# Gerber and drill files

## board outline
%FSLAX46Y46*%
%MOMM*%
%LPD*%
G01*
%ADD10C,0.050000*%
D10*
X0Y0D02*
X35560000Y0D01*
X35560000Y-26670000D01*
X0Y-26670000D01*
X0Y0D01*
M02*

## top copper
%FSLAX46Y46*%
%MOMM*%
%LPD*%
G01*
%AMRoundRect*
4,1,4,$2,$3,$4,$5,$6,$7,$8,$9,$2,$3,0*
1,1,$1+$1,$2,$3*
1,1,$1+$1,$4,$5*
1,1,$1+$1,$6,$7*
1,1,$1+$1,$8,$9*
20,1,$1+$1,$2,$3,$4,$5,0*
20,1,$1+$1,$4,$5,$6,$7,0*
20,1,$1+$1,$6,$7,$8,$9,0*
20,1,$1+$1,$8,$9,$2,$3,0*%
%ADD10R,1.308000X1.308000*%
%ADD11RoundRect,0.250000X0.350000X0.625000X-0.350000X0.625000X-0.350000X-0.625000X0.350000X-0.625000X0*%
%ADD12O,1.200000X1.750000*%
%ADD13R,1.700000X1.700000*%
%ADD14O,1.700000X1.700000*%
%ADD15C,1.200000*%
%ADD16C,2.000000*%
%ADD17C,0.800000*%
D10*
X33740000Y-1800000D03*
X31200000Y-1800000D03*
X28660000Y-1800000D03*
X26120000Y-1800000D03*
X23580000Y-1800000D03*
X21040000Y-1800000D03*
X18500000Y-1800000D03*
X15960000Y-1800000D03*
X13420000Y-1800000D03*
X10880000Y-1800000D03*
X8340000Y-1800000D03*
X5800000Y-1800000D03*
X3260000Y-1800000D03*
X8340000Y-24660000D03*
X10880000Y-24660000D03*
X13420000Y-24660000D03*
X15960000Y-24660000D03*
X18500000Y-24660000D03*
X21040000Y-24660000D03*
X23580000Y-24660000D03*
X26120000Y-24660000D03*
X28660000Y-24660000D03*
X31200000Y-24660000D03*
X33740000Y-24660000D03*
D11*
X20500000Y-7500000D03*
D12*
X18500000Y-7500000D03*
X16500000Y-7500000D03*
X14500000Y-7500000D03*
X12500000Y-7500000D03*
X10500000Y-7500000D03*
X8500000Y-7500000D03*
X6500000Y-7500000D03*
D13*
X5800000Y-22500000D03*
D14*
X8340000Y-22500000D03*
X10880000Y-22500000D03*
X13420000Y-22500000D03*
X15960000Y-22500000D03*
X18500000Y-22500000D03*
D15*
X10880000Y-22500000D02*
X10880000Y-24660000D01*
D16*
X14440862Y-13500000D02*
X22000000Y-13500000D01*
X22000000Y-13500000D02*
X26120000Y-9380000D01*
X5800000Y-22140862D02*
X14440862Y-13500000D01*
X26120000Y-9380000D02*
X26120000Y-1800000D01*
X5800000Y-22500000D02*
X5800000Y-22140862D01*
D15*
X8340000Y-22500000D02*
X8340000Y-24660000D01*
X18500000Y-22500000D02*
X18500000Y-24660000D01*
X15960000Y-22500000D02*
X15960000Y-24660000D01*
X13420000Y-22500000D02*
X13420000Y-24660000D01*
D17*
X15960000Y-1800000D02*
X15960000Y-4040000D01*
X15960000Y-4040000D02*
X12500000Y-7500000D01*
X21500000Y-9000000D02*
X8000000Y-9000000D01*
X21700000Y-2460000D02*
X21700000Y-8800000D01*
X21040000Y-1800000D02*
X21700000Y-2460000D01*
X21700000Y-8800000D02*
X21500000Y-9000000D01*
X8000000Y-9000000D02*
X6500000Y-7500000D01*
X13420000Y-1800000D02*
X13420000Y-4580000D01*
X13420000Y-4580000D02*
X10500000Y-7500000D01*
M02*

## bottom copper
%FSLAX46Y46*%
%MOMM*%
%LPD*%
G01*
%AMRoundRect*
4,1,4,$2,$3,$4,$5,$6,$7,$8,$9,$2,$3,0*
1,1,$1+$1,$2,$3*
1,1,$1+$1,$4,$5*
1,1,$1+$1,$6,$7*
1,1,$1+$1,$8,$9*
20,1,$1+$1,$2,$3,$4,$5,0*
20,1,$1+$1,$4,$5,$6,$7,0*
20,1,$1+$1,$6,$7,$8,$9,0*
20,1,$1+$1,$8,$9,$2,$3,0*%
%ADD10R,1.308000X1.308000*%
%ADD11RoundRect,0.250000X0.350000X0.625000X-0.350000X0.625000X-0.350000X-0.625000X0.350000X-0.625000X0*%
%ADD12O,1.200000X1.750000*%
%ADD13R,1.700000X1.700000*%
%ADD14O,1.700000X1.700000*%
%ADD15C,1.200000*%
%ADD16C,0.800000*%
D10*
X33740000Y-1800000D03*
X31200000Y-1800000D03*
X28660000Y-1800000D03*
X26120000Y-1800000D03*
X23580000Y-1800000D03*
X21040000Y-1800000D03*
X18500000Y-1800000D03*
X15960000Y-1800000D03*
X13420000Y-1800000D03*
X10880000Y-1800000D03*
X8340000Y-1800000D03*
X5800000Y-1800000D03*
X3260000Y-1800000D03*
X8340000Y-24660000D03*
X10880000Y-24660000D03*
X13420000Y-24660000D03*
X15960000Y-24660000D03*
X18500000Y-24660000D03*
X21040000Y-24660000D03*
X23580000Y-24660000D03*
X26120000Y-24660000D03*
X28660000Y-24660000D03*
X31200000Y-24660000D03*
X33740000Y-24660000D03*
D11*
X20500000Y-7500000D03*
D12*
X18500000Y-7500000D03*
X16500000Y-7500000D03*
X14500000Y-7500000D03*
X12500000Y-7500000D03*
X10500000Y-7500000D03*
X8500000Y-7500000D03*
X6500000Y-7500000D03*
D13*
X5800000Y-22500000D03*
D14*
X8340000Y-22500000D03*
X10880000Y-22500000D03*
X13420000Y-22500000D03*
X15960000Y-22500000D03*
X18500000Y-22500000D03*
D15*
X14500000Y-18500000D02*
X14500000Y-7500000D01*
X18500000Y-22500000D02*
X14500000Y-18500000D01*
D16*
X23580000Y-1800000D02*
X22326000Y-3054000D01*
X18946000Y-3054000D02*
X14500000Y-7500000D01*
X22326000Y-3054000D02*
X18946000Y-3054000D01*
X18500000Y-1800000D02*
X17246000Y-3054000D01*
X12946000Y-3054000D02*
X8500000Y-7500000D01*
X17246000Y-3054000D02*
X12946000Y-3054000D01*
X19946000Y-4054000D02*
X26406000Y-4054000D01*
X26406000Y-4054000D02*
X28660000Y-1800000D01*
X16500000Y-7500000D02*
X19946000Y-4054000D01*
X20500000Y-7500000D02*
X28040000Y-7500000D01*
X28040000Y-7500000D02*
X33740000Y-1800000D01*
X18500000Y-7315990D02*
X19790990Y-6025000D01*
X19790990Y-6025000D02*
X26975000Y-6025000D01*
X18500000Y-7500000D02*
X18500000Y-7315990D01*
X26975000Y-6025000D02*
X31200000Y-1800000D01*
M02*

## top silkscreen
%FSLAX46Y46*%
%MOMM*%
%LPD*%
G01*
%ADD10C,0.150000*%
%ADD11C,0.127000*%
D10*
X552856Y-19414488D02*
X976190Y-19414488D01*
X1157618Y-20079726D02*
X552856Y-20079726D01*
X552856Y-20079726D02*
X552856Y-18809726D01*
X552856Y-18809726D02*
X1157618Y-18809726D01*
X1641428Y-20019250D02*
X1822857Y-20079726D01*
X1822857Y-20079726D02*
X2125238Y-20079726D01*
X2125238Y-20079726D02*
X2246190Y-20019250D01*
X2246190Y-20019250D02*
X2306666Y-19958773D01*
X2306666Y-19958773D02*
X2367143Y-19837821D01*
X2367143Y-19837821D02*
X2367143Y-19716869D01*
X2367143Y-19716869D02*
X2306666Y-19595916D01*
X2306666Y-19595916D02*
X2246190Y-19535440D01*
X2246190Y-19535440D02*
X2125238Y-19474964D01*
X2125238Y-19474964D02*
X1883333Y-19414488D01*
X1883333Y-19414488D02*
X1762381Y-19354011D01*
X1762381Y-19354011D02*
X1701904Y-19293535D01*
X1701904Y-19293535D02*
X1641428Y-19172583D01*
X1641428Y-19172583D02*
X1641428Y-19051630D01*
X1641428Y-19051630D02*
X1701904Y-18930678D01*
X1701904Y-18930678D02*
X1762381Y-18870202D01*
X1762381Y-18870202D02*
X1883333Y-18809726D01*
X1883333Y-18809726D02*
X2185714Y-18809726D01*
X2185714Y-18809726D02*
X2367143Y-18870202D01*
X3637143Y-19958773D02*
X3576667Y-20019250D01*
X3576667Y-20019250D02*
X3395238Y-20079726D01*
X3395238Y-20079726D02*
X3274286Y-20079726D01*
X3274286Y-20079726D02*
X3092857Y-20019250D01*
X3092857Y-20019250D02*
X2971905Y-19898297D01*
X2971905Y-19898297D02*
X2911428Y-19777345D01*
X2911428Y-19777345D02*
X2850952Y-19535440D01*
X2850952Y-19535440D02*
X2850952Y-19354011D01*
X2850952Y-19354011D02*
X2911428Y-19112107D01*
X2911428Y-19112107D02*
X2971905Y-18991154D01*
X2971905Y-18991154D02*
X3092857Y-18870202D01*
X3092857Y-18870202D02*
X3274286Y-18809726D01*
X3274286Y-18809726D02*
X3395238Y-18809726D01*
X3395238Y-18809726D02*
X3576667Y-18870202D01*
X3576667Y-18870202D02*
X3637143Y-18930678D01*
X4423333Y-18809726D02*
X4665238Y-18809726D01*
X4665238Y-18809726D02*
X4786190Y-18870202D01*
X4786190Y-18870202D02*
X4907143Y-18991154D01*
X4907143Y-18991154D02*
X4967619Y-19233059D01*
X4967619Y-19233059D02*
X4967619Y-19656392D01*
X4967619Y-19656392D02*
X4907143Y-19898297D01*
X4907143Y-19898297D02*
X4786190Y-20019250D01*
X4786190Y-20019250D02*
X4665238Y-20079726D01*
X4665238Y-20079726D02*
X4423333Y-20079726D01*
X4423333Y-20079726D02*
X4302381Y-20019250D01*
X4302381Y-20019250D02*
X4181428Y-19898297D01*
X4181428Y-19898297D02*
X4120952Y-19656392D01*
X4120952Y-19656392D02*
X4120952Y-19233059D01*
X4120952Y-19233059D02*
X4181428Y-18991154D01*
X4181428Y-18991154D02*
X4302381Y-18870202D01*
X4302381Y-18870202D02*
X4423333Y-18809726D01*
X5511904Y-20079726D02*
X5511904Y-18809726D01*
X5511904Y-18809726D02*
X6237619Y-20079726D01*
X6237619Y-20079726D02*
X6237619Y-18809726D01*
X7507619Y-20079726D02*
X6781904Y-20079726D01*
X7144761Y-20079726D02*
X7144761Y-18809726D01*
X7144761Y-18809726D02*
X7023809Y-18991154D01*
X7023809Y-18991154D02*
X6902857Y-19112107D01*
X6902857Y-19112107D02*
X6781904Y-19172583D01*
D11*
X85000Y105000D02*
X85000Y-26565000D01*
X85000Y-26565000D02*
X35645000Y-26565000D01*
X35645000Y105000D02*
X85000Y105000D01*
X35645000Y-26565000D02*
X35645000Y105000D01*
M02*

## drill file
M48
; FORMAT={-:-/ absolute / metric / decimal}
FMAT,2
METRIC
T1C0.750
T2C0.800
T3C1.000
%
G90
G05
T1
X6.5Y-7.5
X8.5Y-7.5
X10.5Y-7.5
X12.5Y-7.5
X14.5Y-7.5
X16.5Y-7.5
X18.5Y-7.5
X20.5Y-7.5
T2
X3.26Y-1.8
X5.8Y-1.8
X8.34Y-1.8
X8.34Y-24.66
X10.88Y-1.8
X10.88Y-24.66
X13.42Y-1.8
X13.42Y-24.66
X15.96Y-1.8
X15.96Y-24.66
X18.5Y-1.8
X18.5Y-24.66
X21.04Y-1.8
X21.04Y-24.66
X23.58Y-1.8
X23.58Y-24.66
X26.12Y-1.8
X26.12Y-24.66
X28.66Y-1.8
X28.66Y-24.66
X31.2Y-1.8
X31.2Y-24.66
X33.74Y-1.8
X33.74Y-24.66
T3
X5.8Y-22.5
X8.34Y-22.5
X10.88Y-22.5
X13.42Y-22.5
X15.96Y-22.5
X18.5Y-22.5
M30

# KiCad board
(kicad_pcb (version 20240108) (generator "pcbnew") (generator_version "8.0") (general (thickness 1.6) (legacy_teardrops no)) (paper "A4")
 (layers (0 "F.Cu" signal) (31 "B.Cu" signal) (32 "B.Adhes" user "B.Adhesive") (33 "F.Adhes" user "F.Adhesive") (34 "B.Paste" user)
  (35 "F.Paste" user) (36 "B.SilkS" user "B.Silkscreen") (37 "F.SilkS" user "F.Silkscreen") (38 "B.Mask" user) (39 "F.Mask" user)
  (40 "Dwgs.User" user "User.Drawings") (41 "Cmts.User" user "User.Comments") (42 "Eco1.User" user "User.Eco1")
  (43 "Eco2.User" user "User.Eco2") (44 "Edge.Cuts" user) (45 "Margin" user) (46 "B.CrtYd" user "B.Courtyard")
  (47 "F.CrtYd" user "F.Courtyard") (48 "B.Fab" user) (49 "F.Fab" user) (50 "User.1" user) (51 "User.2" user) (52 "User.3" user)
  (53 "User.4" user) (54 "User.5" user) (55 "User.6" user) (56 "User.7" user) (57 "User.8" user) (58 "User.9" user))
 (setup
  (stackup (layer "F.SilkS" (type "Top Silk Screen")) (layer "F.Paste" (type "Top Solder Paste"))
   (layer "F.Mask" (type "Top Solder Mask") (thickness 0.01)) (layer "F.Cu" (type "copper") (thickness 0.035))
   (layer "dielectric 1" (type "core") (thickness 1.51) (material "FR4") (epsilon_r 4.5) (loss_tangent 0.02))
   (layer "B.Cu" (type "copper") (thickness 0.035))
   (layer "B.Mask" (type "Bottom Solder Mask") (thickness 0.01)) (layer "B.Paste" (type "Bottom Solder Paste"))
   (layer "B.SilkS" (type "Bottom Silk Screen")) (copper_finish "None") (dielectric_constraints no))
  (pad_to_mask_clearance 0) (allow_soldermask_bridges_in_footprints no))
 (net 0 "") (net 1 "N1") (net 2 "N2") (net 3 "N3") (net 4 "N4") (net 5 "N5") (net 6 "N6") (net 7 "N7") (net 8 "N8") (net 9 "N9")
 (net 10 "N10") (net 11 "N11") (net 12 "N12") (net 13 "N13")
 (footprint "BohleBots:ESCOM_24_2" (layer "F.Cu") (at 18.5 14.5)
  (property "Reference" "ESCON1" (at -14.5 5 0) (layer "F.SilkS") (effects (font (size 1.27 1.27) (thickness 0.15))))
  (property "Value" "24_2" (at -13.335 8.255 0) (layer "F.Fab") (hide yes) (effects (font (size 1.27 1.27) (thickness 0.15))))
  (fp_line (start -18.415 -14.605) (end -18.415 12.065) (stroke (width 0.127) (type solid)) (layer "F.SilkS"))
  (fp_line (start -18.415 12.065) (end 17.145 12.065) (stroke (width 0.127) (type solid)) (layer "F.SilkS"))
  (fp_line (start 17.145 -14.605) (end -18.415 -14.605) (stroke (width 0.127) (type solid)) (layer "F.SilkS"))
  (fp_line (start 17.145 12.065) (end 17.145 -14.605) (stroke (width 0.127) (type solid)) (layer "F.SilkS"))
  (pad "P1" thru_hole rect (at 15.24 -12.7) (size 1.308 1.308) (drill 0.8) (layers "*.Cu" "*.Mask") (remove_unused_layers no) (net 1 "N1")
   (thermal_bridge_angle 45))
  (pad "P2" thru_hole rect (at 12.7 -12.7) (size 1.308 1.308) (drill 0.8) (layers "*.Cu" "*.Mask") (remove_unused_layers no) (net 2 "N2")
   (thermal_bridge_angle 45))
  (pad "P3" thru_hole rect (at 10.16 -12.7) (size 1.308 1.308) (drill 0.8) (layers "*.Cu" "*.Mask") (remove_unused_layers no) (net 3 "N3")
   (thermal_bridge_angle 45))
  (pad "P4" thru_hole rect (at 7.62 -12.7) (size 1.308 1.308) (drill 0.8) (layers "*.Cu" "*.Mask") (remove_unused_layers no) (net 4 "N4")
   (thermal_bridge_angle 45))
  (pad "P5" thru_hole rect (at 5.08 -12.7) (size 1.308 1.308) (drill 0.8) (layers "*.Cu" "*.Mask") (remove_unused_layers no) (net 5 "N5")
   (thermal_bridge_angle 45))
  (pad "P6" thru_hole rect (at 2.54 -12.7) (size 1.308 1.308) (drill 0.8) (layers "*.Cu" "*.Mask") (remove_unused_layers no) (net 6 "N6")
   (thermal_bridge_angle 45))
  (pad "P7" thru_hole rect (at 0 -12.7) (size 1.308 1.308) (drill 0.8) (layers "*.Cu" "*.Mask") (remove_unused_layers no) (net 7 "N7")
   (thermal_bridge_angle 45))
  (pad "P8" thru_hole rect (at -2.54 -12.7) (size 1.308 1.308) (drill 0.8) (layers "*.Cu" "*.Mask") (remove_unused_layers no) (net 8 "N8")
   (thermal_bridge_angle 45))
  (pad "P9" thru_hole rect (at -5.08 -12.7) (size 1.308 1.308) (drill 0.8) (layers "*.Cu" "*.Mask") (remove_unused_layers no) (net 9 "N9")
   (thermal_bridge_angle 45))
  (pad "P10" thru_hole rect (at -7.62 -12.7) (size 1.308 1.308) (drill 0.8) (layers "*.Cu" "*.Mask") (remove_unused_layers no)
   (thermal_bridge_angle 45))
  (pad "P11" thru_hole rect (at -10.16 -12.7) (size 1.308 1.308) (drill 0.8) (layers "*.Cu" "*.Mask") (remove_unused_layers no)
   (thermal_bridge_angle 45))
  (pad "P12" thru_hole rect (at -12.7 -12.7) (size 1.308 1.308) (drill 0.8) (layers "*.Cu" "*.Mask") (remove_unused_layers no)
   (thermal_bridge_angle 45))
  (pad "P13" thru_hole rect (at -15.24 -12.7) (size 1.308 1.308) (drill 0.8) (layers "*.Cu" "*.Mask") (remove_unused_layers no)
   (thermal_bridge_angle 45))
  (pad "P14" thru_hole rect (at -10.16 10.16) (size 1.308 1.308) (drill 0.8) (layers "*.Cu" "*.Mask") (remove_unused_layers no)
   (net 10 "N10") (thermal_bridge_angle 45))
  (pad "P15" thru_hole rect (at -7.62 10.16) (size 1.308 1.308) (drill 0.8) (layers "*.Cu" "*.Mask") (remove_unused_layers no)
   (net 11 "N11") (thermal_bridge_angle 45))
  (pad "P16" thru_hole rect (at -5.08 10.16) (size 1.308 1.308) (drill 0.8) (layers "*.Cu" "*.Mask") (remove_unused_layers no)
   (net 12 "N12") (thermal_bridge_angle 45))
  (pad "P17" thru_hole rect (at -2.54 10.16) (size 1.308 1.308) (drill 0.8) (layers "*.Cu" "*.Mask") (remove_unused_layers no)
   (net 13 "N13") (thermal_bridge_angle 45))
  (pad "P18" thru_hole rect (at 0 10.16) (size 1.308 1.308) (drill 0.8) (layers "*.Cu" "*.Mask") (remove_unused_layers no) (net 5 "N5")
   (thermal_bridge_angle 45))
  (pad "P19" thru_hole rect (at 2.54 10.16) (size 1.308 1.308) (drill 0.8) (layers "*.Cu" "*.Mask") (remove_unused_layers no)
   (thermal_bridge_angle 45))
  (pad "P20" thru_hole rect (at 5.08 10.16) (size 1.308 1.308) (drill 0.8) (layers "*.Cu" "*.Mask") (remove_unused_layers no)
   (thermal_bridge_angle 45))
  (pad "P21" thru_hole rect (at 7.62 10.16) (size 1.308 1.308) (drill 0.8) (layers "*.Cu" "*.Mask") (remove_unused_layers no)
   (thermal_bridge_angle 45))
  (pad "P22" thru_hole rect (at 10.16 10.16) (size 1.308 1.308) (drill 0.8) (layers "*.Cu" "*.Mask") (remove_unused_layers no)
   (thermal_bridge_angle 45))
  (pad "P23" thru_hole rect (at 12.7 10.16) (size 1.308 1.308) (drill 0.8) (layers "*.Cu" "*.Mask") (remove_unused_layers no)
   (thermal_bridge_angle 45))
  (pad "P24" thru_hole rect (at 15.24 10.16) (size 1.308 1.308) (drill 0.8) (layers "*.Cu" "*.Mask") (remove_unused_layers no)
   (thermal_bridge_angle 45)))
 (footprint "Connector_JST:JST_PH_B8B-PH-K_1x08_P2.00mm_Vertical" (layer "B.Cu") (at 20.5 7.5 180)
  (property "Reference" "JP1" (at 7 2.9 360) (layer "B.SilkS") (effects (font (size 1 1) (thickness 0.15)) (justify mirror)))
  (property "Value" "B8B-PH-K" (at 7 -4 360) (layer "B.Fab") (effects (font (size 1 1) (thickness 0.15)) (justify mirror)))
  (pad "1" thru_hole roundrect (at 0 0 180) (size 1.2 1.75) (drill 0.75) (layers "*.Cu" "*.Mask") (remove_unused_layers no)
   (roundrect_rratio 0.208333) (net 1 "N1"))
  (pad "2" thru_hole oval (at 2 0 180) (size 1.2 1.75) (drill 0.75) (layers "*.Cu" "*.Mask") (remove_unused_layers no) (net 2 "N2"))
  (pad "3" thru_hole oval (at 4 0 180) (size 1.2 1.75) (drill 0.75) (layers "*.Cu" "*.Mask") (remove_unused_layers no) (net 3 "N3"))
  (pad "4" thru_hole oval (at 6 0 180) (size 1.2 1.75) (drill 0.75) (layers "*.Cu" "*.Mask") (remove_unused_layers no) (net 5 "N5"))
  (pad "5" thru_hole oval (at 8 0 180) (size 1.2 1.75) (drill 0.75) (layers "*.Cu" "*.Mask") (remove_unused_layers no) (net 8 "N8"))
  (pad "6" thru_hole oval (at 10 0 180) (size 1.2 1.75) (drill 0.75) (layers "*.Cu" "*.Mask") (remove_unused_layers no) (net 9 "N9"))
  (pad "7" thru_hole oval (at 12 0 180) (size 1.2 1.75) (drill 0.75) (layers "*.Cu" "*.Mask") (remove_unused_layers no) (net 7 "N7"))
  (pad "8" thru_hole oval (at 14 0 180) (size 1.2 1.75) (drill 0.75) (layers "*.Cu" "*.Mask") (remove_unused_layers no) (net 6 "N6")))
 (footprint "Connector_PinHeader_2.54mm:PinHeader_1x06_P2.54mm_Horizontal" (layer "B.Cu") (at 5.8 22.5 -90)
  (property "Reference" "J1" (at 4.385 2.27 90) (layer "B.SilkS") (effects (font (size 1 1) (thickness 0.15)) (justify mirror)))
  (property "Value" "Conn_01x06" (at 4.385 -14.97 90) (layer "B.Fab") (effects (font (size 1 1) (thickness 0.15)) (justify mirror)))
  (pad "1" thru_hole rect (at 0 0 270) (size 1.7 1.7) (drill 1) (layers "*.Cu" "*.Mask") (remove_unused_layers no) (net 4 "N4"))
  (pad "2" thru_hole oval (at 0 -2.54 270) (size 1.7 1.7) (drill 1) (layers "*.Cu" "*.Mask") (remove_unused_layers no) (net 10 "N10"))
  (pad "3" thru_hole oval (at 0 -5.08 270) (size 1.7 1.7) (drill 1) (layers "*.Cu" "*.Mask") (remove_unused_layers no) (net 11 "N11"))
  (pad "4" thru_hole oval (at 0 -7.62 270) (size 1.7 1.7) (drill 1) (layers "*.Cu" "*.Mask") (remove_unused_layers no) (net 12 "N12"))
  (pad "5" thru_hole oval (at 0 -10.16 270) (size 1.7 1.7) (drill 1) (layers "*.Cu" "*.Mask") (remove_unused_layers no) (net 13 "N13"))
  (pad "6" thru_hole oval (at 0 -12.7 270) (size 1.7 1.7) (drill 1) (layers "*.Cu" "*.Mask") (remove_unused_layers no) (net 5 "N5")))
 (gr_rect (start 0 0) (end 35.56 26.67) (stroke (width 0.05) (type default)) (fill none) (layer "Edge.Cuts"))
 (segment (start 10.88 22.5) (end 10.88 24.66) (width 1.2) (layer "F.Cu") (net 11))
 (segment (start 14.440862 13.5) (end 22 13.5) (width 2) (layer "F.Cu") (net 4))
 (segment (start 22 13.5) (end 26.12 9.38) (width 2) (layer "F.Cu") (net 4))
 (segment (start 5.8 22.140862) (end 14.440862 13.5) (width 2) (layer "F.Cu") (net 4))
 (segment (start 26.12 9.38) (end 26.12 1.8) (width 2) (layer "F.Cu") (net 4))
 (segment (start 5.8 22.5) (end 5.8 22.140862) (width 2) (layer "F.Cu") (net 4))
 (segment (start 8.34 22.5) (end 8.34 24.66) (width 1.2) (layer "F.Cu") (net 10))
 (segment (start 18.5 22.5) (end 18.5 24.66) (width 1.2) (layer "F.Cu") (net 5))
 (segment (start 14.5 18.5) (end 14.5 7.5) (width 1.2) (layer "B.Cu") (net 5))
 (segment (start 18.5 22.5) (end 14.5 18.5) (width 1.2) (layer "B.Cu") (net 5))
 (segment (start 23.58 1.8) (end 22.326 3.054) (width 0.8) (layer "B.Cu") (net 5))
 (segment (start 18.946 3.054) (end 14.5 7.5) (width 0.8) (layer "B.Cu") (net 5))
 (segment (start 22.326 3.054) (end 18.946 3.054) (width 0.8) (layer "B.Cu") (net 5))
 (segment (start 15.96 22.5) (end 15.96 24.66) (width 1.2) (layer "F.Cu") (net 13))
 (segment (start 13.42 22.5) (end 13.42 24.66) (width 1.2) (layer "F.Cu") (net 12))
 (segment (start 18.5 1.8) (end 17.246 3.054) (width 0.8) (layer "B.Cu") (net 7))
 (segment (start 12.946 3.054) (end 8.5 7.5) (width 0.8) (layer "B.Cu") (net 7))
 (segment (start 17.246 3.054) (end 12.946 3.054) (width 0.8) (layer "B.Cu") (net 7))
 (segment (start 15.96 1.8) (end 15.96 4.04) (width 0.8) (layer "F.Cu") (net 8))
 (segment (start 15.96 4.04) (end 12.5 7.5) (width 0.8) (layer "F.Cu") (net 8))
 (segment (start 19.946 4.054) (end 26.406 4.054) (width 0.8) (layer "B.Cu") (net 3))
 (segment (start 26.406 4.054) (end 28.66 1.8) (width 0.8) (layer "B.Cu") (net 3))
 (segment (start 16.5 7.5) (end 19.946 4.054) (width 0.8) (layer "B.Cu") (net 3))
 (segment (start 21.5 9) (end 8 9) (width 0.8) (layer "F.Cu") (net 6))
 (segment (start 21.7 2.46) (end 21.7 8.8) (width 0.8) (layer "F.Cu") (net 6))
 (segment (start 21.04 1.8) (end 21.7 2.46) (width 0.8) (layer "F.Cu") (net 6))
 (segment (start 21.7 8.8) (end 21.5 9) (width 0.8) (layer "F.Cu") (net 6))
 (segment (start 8 9) (end 6.5 7.5) (width 0.8) (layer "F.Cu") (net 6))
 (segment (start 20.5 7.5) (end 28.04 7.5) (width 0.8) (layer "B.Cu") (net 1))
 (segment (start 28.04 7.5) (end 33.74 1.8) (width 0.8) (layer "B.Cu") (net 1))
 (segment (start 13.42 1.8) (end 13.42 4.58) (width 0.8) (layer "F.Cu") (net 9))
 (segment (start 13.42 4.58) (end 10.5 7.5) (width 0.8) (layer "F.Cu") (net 9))
 (segment (start 18.5 7.31599) (end 19.79099 6.025) (width 0.8) (layer "B.Cu") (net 2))
 (segment (start 19.79099 6.025) (end 26.975 6.025) (width 0.8) (layer "B.Cu") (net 2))
 (segment (start 18.5 7.5) (end 18.5 7.31599) (width 0.8) (layer "B.Cu") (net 2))
 (segment (start 26.975 6.025) (end 31.2 1.8) (width 0.8) (layer "B.Cu") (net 2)))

